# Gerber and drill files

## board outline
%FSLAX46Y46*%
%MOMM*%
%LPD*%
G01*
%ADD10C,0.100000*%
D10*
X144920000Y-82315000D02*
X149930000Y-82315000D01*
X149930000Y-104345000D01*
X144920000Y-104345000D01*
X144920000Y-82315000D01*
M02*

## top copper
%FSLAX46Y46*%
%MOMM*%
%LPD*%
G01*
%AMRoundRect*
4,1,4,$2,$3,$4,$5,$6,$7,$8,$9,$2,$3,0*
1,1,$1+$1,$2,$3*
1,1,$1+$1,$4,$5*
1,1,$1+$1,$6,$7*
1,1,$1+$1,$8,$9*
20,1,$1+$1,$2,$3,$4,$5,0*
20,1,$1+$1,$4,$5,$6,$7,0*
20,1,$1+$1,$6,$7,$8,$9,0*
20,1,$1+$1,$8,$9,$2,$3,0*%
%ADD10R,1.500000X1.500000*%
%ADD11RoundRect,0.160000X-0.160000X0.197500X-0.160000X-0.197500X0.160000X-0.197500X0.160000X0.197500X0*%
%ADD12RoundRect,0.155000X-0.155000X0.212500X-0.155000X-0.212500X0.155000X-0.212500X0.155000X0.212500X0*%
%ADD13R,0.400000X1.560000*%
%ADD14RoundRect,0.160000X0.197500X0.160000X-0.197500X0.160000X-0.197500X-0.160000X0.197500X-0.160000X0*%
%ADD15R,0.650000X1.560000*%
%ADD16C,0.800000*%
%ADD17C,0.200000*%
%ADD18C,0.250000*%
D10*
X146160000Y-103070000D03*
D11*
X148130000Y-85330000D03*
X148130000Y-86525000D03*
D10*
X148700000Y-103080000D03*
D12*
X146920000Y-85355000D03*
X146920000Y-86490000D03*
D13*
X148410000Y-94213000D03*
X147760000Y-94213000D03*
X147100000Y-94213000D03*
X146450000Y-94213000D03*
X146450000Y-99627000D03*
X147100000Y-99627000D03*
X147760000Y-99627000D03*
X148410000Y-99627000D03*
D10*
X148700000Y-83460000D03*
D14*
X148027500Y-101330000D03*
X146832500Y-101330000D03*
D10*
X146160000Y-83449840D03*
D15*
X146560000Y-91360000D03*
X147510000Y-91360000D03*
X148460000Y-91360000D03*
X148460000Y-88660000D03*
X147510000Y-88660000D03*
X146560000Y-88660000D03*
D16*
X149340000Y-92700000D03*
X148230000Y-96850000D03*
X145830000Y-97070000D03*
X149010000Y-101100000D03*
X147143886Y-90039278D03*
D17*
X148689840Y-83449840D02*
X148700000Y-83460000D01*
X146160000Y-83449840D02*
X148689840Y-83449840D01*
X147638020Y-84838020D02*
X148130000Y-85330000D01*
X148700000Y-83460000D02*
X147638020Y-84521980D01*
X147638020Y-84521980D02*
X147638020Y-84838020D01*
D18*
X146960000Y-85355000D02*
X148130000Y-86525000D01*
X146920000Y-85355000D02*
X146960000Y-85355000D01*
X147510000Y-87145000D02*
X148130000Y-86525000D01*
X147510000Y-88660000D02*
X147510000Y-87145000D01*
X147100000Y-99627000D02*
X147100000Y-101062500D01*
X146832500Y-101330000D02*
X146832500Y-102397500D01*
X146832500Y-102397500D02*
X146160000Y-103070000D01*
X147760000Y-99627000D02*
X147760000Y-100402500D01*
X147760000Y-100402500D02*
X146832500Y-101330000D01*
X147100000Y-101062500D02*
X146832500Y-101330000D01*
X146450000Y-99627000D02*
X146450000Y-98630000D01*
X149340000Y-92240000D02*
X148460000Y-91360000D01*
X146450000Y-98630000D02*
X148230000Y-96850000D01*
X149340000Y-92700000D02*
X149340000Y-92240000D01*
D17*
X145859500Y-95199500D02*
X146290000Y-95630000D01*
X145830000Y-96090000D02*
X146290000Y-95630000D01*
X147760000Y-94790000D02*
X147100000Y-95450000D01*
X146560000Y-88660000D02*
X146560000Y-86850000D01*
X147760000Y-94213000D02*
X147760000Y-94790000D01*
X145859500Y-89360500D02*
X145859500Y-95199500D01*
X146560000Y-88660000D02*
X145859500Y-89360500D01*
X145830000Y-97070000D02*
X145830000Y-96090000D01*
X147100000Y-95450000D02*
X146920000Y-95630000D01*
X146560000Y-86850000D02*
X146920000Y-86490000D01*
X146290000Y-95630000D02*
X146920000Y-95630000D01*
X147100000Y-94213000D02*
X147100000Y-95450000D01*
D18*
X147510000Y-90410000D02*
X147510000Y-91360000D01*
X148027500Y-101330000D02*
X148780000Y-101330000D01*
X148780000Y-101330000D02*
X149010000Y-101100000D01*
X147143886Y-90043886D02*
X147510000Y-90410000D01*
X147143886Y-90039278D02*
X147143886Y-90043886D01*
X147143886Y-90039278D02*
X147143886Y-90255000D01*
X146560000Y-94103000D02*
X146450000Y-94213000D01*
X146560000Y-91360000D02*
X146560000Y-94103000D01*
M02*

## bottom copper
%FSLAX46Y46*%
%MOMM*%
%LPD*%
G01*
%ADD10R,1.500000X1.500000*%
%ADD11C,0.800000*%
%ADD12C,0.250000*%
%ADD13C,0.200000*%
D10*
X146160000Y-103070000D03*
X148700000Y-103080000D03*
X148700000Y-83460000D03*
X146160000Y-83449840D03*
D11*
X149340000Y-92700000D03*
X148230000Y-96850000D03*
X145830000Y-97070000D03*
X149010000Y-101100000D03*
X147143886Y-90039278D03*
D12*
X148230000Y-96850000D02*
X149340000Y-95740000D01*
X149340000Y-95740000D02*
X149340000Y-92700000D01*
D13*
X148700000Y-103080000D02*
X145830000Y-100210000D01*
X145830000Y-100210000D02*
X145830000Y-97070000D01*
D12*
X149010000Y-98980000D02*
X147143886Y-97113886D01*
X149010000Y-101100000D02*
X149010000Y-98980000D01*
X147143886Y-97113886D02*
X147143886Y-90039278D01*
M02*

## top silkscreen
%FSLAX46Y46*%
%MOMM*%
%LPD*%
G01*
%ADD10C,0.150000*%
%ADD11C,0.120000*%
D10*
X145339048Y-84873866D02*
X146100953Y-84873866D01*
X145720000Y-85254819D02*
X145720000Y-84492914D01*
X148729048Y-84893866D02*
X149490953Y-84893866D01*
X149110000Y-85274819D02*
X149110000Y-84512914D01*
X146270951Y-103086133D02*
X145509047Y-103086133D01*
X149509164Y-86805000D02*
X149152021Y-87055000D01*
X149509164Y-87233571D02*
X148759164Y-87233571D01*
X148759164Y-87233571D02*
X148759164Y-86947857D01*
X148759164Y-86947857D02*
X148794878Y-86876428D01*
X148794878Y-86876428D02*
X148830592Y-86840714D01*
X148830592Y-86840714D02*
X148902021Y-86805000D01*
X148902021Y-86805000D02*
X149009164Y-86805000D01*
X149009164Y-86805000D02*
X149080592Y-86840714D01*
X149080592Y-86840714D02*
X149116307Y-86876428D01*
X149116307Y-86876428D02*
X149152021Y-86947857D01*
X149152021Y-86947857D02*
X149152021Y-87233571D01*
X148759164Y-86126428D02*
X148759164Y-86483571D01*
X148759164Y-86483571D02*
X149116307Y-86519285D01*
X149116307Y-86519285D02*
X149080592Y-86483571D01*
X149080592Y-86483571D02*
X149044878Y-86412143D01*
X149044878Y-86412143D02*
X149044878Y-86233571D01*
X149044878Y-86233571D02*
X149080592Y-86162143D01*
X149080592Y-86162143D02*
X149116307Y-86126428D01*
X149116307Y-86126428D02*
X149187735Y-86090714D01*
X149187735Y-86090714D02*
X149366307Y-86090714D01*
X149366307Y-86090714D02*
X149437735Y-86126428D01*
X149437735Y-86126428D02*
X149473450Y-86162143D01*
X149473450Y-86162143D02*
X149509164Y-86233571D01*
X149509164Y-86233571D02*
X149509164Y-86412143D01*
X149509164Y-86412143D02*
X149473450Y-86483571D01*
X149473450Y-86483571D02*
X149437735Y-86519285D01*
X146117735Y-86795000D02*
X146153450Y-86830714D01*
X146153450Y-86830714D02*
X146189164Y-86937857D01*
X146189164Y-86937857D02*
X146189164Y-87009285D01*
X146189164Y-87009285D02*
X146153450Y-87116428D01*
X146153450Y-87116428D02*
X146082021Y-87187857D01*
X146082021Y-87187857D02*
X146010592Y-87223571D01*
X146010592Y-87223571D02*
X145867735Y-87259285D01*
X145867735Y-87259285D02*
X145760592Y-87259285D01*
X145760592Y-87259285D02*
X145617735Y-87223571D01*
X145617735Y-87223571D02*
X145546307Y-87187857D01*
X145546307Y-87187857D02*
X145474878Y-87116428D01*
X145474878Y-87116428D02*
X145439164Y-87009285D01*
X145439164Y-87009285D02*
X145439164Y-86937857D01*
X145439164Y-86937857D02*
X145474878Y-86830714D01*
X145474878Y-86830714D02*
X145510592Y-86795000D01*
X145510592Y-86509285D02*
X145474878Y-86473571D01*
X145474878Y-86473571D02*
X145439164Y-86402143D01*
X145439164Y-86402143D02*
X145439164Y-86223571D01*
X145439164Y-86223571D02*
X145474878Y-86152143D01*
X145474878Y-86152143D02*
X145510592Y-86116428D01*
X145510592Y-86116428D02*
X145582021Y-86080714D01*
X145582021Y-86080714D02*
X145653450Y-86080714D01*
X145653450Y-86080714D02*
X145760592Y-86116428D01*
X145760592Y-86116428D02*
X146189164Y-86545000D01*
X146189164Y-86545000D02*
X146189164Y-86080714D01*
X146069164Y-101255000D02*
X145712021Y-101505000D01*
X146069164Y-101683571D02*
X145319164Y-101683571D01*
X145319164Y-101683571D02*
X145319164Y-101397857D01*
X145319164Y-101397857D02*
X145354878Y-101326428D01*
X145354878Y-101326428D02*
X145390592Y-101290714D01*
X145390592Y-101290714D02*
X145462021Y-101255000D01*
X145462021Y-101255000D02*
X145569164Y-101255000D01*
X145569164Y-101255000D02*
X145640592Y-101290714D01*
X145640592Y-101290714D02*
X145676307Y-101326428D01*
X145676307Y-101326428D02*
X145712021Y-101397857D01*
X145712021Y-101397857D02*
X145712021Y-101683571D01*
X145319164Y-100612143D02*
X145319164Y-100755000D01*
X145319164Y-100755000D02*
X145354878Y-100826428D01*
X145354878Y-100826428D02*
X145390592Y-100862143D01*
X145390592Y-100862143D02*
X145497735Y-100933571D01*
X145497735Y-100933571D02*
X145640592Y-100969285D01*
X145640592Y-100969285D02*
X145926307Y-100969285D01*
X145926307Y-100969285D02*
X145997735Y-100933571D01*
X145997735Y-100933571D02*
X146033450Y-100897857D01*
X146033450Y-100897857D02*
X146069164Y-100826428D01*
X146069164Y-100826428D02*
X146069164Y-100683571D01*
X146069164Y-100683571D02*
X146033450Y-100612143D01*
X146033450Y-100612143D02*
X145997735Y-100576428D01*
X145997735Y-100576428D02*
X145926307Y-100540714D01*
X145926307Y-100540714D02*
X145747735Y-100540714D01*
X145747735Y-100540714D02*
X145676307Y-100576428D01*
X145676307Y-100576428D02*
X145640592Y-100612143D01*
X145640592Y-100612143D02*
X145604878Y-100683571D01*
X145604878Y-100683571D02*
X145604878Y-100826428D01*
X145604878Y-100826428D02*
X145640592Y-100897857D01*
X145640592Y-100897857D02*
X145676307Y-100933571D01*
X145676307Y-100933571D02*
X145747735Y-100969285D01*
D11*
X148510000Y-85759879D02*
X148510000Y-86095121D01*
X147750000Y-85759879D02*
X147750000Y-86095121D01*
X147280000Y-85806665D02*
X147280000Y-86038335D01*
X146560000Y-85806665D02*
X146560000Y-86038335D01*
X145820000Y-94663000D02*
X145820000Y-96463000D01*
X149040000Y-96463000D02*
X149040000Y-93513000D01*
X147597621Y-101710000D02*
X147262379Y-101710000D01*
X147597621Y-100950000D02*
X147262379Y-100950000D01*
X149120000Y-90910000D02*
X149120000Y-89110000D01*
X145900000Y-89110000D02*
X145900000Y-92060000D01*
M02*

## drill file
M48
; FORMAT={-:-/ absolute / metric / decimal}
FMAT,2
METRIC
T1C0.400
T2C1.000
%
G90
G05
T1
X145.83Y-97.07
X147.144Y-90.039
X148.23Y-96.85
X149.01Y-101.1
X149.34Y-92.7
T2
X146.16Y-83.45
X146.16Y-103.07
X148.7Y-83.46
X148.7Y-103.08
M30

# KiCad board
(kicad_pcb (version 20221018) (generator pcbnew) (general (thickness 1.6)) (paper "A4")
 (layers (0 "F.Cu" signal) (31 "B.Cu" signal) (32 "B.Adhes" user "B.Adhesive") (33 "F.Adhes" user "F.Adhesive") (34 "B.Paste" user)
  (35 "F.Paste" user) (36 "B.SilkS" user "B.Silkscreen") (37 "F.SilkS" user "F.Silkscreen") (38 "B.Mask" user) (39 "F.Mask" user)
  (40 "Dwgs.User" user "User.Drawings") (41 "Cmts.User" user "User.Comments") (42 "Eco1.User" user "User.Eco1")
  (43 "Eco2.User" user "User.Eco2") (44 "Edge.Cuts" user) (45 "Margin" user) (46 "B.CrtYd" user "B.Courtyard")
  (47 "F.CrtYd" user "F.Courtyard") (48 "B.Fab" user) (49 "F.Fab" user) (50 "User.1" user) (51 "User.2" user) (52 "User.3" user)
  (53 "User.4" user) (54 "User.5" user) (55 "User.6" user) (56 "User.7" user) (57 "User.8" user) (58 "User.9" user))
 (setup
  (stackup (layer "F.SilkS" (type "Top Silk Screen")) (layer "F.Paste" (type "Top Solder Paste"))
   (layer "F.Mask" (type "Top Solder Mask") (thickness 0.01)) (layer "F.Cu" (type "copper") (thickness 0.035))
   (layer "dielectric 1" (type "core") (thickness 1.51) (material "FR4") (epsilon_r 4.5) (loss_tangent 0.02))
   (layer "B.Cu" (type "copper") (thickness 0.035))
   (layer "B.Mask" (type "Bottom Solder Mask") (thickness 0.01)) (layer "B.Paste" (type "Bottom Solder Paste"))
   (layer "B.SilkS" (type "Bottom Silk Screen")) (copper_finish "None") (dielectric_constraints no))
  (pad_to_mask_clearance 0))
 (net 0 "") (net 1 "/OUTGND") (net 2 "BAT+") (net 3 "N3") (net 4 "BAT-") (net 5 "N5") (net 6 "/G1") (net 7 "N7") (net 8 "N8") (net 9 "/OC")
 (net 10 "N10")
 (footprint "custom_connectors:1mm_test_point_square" (layer "F.Cu") (at 146.16 103.08016)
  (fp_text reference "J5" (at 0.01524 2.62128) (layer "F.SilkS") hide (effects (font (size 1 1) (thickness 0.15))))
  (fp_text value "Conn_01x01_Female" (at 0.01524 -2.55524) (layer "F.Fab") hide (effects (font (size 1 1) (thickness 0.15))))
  (pad "1" thru_hole rect (at 0 -0.01016) (size 1.5 1.5) (drill 1) (layers "*.Cu" "*.Mask") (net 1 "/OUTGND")))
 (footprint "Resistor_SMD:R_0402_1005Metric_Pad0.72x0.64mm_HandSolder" (layer "F.Cu") (at 148.13 85.9275 -90)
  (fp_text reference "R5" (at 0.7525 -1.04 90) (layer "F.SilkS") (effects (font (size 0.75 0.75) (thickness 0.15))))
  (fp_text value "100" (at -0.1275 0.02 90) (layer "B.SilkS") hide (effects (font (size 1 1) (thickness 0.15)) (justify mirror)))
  (fp_line (start -0.167621 -0.38) (end 0.167621 -0.38) (stroke (width 0.12) (type solid)) (layer "F.SilkS"))
  (fp_line (start -0.167621 0.38) (end 0.167621 0.38) (stroke (width 0.12) (type solid)) (layer "F.SilkS"))
  (pad "1" smd roundrect (at -0.5975 0 270) (size 0.715 0.64) (layers "F.Cu" "F.Paste" "F.Mask") (roundrect_rratio 0.25) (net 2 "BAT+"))
  (pad "2" smd roundrect (at 0.5975 0 270) (size 0.715 0.64) (layers "F.Cu" "F.Paste" "F.Mask") (roundrect_rratio 0.25) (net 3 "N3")))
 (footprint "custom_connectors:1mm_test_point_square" (layer "F.Cu") (at 148.7 103.09016)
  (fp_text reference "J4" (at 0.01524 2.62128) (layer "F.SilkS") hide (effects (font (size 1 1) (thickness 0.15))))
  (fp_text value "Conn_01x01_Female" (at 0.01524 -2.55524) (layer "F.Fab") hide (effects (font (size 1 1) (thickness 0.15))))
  (pad "1" thru_hole rect (at 0 -0.01016) (size 1.5 1.5) (drill 1) (layers "*.Cu" "*.Mask") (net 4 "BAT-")))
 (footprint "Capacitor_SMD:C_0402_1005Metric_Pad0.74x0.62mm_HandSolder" (layer "F.Cu") (at 146.92 85.9225 -90)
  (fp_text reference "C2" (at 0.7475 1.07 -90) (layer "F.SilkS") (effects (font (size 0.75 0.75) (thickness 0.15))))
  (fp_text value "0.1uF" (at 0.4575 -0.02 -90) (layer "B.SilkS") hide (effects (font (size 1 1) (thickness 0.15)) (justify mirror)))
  (fp_line (start -0.115835 -0.36) (end 0.115835 -0.36) (stroke (width 0.12) (type solid)) (layer "F.SilkS"))
  (fp_line (start -0.115835 0.36) (end 0.115835 0.36) (stroke (width 0.12) (type solid)) (layer "F.SilkS"))
  (pad "1" smd roundrect (at -0.5675 0 270) (size 0.735 0.62) (layers "F.Cu" "F.Paste" "F.Mask") (roundrect_rratio 0.25) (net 3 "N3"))
  (pad "2" smd roundrect (at 0.5675 0 270) (size 0.735 0.62) (layers "F.Cu" "F.Paste" "F.Mask") (roundrect_rratio 0.25) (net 4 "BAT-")))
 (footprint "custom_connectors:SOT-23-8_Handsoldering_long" (layer "F.Cu") (at 147.43 95.563 -90)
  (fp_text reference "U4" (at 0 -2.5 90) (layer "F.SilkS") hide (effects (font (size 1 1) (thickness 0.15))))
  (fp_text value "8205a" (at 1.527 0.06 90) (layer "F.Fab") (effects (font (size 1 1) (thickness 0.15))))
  (fp_line (start -0.9 1.61) (end 0.9 1.61) (stroke (width 0.12) (type solid)) (layer "F.SilkS"))
  (fp_line (start 0.9 -1.61) (end -2.05 -1.61) (stroke (width 0.12) (type solid)) (layer "F.SilkS"))
  (pad "1" smd rect (at -1.35 -0.98 270) (size 1.56 0.4) (layers "F.Cu" "F.Paste" "F.Mask") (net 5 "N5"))
  (pad "2" smd rect (at -1.35 -0.33 270) (size 1.56 0.4) (layers "F.Cu" "F.Paste" "F.Mask") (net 4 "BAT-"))
  (pad "3" smd rect (at -1.35 0.33 270) (size 1.56 0.4) (layers "F.Cu" "F.Paste" "F.Mask") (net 4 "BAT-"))
  (pad "4" smd rect (at -1.35 0.98 270) (size 1.56 0.4) (layers "F.Cu" "F.Paste" "F.Mask") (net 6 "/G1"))
  (pad "5" smd rect (at 4.064 0.98 270) (size 1.56 0.4) (layers "F.Cu" "F.Paste" "F.Mask") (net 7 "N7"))
  (pad "6" smd rect (at 4.064 0.33 270) (size 1.56 0.4) (layers "F.Cu" "F.Paste" "F.Mask") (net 1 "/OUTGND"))
  (pad "7" smd rect (at 4.064 -0.33 270) (size 1.56 0.4) (layers "F.Cu" "F.Paste" "F.Mask") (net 1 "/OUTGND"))
  (pad "8" smd rect (at 4.064 -0.98 270) (size 1.56 0.4) (layers "F.Cu" "F.Paste" "F.Mask") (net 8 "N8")))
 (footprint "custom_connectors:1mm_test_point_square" (layer "F.Cu") (at 148.7 83.47016)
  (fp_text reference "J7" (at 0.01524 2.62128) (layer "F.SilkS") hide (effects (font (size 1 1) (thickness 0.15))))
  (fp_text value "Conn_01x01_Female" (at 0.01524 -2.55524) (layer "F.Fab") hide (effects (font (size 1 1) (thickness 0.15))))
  (pad "1" thru_hole rect (at 0 -0.01016) (size 1.5 1.5) (drill 1) (layers "*.Cu" "*.Mask") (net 2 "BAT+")))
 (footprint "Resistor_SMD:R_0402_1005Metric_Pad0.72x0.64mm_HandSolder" (layer "F.Cu") (at 147.43 101.33 180)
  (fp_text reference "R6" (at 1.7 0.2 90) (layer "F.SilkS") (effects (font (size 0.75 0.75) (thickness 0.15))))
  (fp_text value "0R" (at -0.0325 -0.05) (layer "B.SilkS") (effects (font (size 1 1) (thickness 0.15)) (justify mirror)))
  (fp_line (start -0.167621 -0.38) (end 0.167621 -0.38) (stroke (width 0.12) (type solid)) (layer "F.SilkS"))
  (fp_line (start -0.167621 0.38) (end 0.167621 0.38) (stroke (width 0.12) (type solid)) (layer "F.SilkS"))
  (pad "1" smd roundrect (at -0.5975 0 180) (size 0.715 0.64) (layers "F.Cu" "F.Paste" "F.Mask") (roundrect_rratio 0.25) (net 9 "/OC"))
  (pad "2" smd roundrect (at 0.5975 0 180) (size 0.715 0.64) (layers "F.Cu" "F.Paste" "F.Mask") (roundrect_rratio 0.25) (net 1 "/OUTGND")))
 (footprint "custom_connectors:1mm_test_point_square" (layer "F.Cu") (at 146.16 83.46)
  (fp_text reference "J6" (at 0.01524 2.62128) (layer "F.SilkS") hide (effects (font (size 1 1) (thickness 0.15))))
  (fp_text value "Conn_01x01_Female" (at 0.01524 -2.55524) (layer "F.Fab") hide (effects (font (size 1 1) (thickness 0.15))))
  (pad "1" thru_hole rect (at 0 -0.01016) (size 1.5 1.5) (drill 1) (layers "*.Cu" "*.Mask") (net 2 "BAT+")))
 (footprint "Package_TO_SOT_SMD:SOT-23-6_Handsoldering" (layer "F.Cu") (at 147.51 90.01 90)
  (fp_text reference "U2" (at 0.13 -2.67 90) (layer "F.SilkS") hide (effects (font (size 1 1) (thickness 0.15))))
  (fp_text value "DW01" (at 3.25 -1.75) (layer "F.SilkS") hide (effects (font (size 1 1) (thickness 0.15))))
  (fp_line (start -0.9 1.61) (end 0.9 1.61) (stroke (width 0.12) (type solid)) (layer "F.SilkS"))
  (fp_line (start 0.9 -1.61) (end -2.05 -1.61) (stroke (width 0.12) (type solid)) (layer "F.SilkS"))
  (pad "1" smd rect (at -1.35 -0.95 90) (size 1.56 0.65) (layers "F.Cu" "F.Paste" "F.Mask") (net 6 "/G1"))
  (pad "2" smd rect (at -1.35 0 90) (size 1.56 0.65) (layers "F.Cu" "F.Paste" "F.Mask") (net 9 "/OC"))
  (pad "3" smd rect (at -1.35 0.95 90) (size 1.56 0.65) (layers "F.Cu" "F.Paste" "F.Mask") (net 7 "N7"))
  (pad "4" smd rect (at 1.35 0.95 90) (size 1.56 0.65) (layers "F.Cu" "F.Paste" "F.Mask") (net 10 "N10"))
  (pad "5" smd rect (at 1.35 0 90) (size 1.56 0.65) (layers "F.Cu" "F.Paste" "F.Mask") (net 3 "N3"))
  (pad "6" smd rect (at 1.35 -0.95 90) (size 1.56 0.65) (layers "F.Cu" "F.Paste" "F.Mask") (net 4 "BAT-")))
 (gr_rect (start 144.92 82.315) (end 149.93 104.345) (stroke (width 0.1) (type default)) (fill none) (layer "Edge.Cuts"))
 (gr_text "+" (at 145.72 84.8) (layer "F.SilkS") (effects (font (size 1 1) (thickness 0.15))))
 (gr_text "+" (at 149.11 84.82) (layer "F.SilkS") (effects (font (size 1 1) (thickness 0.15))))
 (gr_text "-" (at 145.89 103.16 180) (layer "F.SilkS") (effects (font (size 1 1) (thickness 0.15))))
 (segment (start 148.68984 83.44984) (end 148.7 83.46) (width 0.2) (layer "F.Cu") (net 2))
 (segment (start 146.16 83.44984) (end 148.68984 83.44984) (width 0.2) (layer "F.Cu") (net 2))
 (segment (start 147.63802 84.83802) (end 148.13 85.33) (width 0.2) (layer "F.Cu") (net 2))
 (segment (start 148.7 83.46) (end 147.63802 84.52198) (width 0.2) (layer "F.Cu") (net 2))
 (segment (start 147.63802 84.52198) (end 147.63802 84.83802) (width 0.2) (layer "F.Cu") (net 2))
 (segment (start 146.96 85.355) (end 148.13 86.525) (width 0.25) (layer "F.Cu") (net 3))
 (segment (start 146.92 85.355) (end 146.96 85.355) (width 0.25) (layer "F.Cu") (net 3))
 (segment (start 147.51 87.145) (end 148.13 86.525) (width 0.25) (layer "F.Cu") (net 3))
 (segment (start 147.51 88.66) (end 147.51 87.145) (width 0.25) (layer "F.Cu") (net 3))
 (segment (start 147.1 99.627) (end 147.1 101.0625) (width 0.25) (layer "F.Cu") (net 1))
 (segment (start 146.8325 101.33) (end 146.8325 102.3975) (width 0.25) (layer "F.Cu") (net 1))
 (segment (start 146.8325 102.3975) (end 146.16 103.07) (width 0.25) (layer "F.Cu") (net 1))
 (segment (start 147.76 99.627) (end 147.76 100.4025) (width 0.25) (layer "F.Cu") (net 1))
 (segment (start 147.76 100.4025) (end 146.8325 101.33) (width 0.25) (layer "F.Cu") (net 1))
 (segment (start 147.1 101.0625) (end 146.8325 101.33) (width 0.25) (layer "F.Cu") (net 1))
 (segment (start 146.45 99.627) (end 146.45 98.63) (width 0.25) (layer "F.Cu") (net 7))
 (segment (start 149.34 92.24) (end 148.46 91.36) (width 0.25) (layer "F.Cu") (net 7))
 (segment (start 146.45 98.63) (end 148.23 96.85) (width 0.25) (layer "F.Cu") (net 7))
 (segment (start 149.34 92.7) (end 149.34 92.24) (width 0.25) (layer "F.Cu") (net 7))
 (via (at 149.34 92.7) (size 0.8) (drill 0.4) (layers "F.Cu" "B.Cu") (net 7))
 (via (at 148.23 96.85) (size 0.8) (drill 0.4) (layers "F.Cu" "B.Cu") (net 7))
 (segment (start 148.23 96.85) (end 149.34 95.74) (width 0.25) (layer "B.Cu") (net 7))
 (segment (start 149.34 95.74) (end 149.34 92.7) (width 0.25) (layer "B.Cu") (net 7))
 (segment (start 145.8595 95.1995) (end 146.29 95.63) (width 0.2) (layer "F.Cu") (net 4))
 (segment (start 145.83 96.09) (end 146.29 95.63) (width 0.2) (layer "F.Cu") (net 4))
 (segment (start 147.76 94.79) (end 147.1 95.45) (width 0.2) (layer "F.Cu") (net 4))
 (segment (start 146.56 88.66) (end 146.56 86.85) (width 0.2) (layer "F.Cu") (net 4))
 (segment (start 147.76 94.213) (end 147.76 94.79) (width 0.2) (layer "F.Cu") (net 4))
 (segment (start 145.8595 89.3605) (end 145.8595 95.1995) (width 0.2) (layer "F.Cu") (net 4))
 (segment (start 146.56 88.66) (end 145.8595 89.3605) (width 0.2) (layer "F.Cu") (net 4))
 (segment (start 145.83 97.07) (end 145.83 96.09) (width 0.2) (layer "F.Cu") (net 4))
 (segment (start 147.1 95.45) (end 146.92 95.63) (width 0.2) (layer "F.Cu") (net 4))
 (segment (start 146.56 86.85) (end 146.92 86.49) (width 0.2) (layer "F.Cu") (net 4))
 (segment (start 146.29 95.63) (end 146.92 95.63) (width 0.2) (layer "F.Cu") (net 4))
 (segment (start 147.1 94.213) (end 147.1 95.45) (width 0.2) (layer "F.Cu") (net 4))
 (via (at 145.83 97.07) (size 0.8) (drill 0.4) (layers "F.Cu" "B.Cu") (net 4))
 (segment (start 148.7 103.08) (end 145.83 100.21) (width 0.2) (layer "B.Cu") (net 4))
 (segment (start 145.83 100.21) (end 145.83 97.07) (width 0.2) (layer "B.Cu") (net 4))
 (segment (start 147.51 90.41) (end 147.51 91.36) (width 0.25) (layer "F.Cu") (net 9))
 (segment (start 148.0275 101.33) (end 148.78 101.33) (width 0.25) (layer "F.Cu") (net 9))
 (segment (start 148.78 101.33) (end 149.01 101.1) (width 0.25) (layer "F.Cu") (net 9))
 (segment (start 147.143886 90.043886) (end 147.51 90.41) (width 0.25) (layer "F.Cu") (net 9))
 (segment (start 147.143886 90.039278) (end 147.143886 90.043886) (width 0.25) (layer "F.Cu") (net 9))
 (segment (start 147.143886 90.039278) (end 147.143886 90.255) (width 0.25) (layer "F.Cu") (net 9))
 (via (at 149.01 101.1) (size 0.8) (drill 0.4) (layers "F.Cu" "B.Cu") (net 9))
 (via (at 147.143886 90.039278) (size 0.8) (drill 0.4) (layers "F.Cu" "B.Cu") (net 9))
 (segment (start 149.01 98.98) (end 147.143886 97.113886) (width 0.25) (layer "B.Cu") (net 9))
 (segment (start 149.01 101.1) (end 149.01 98.98) (width 0.25) (layer "B.Cu") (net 9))
 (segment (start 147.143886 97.113886) (end 147.143886 90.039278) (width 0.25) (layer "B.Cu") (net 9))
 (segment (start 146.56 94.103) (end 146.45 94.213) (width 0.25) (layer "F.Cu") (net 6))
 (segment (start 146.56 91.36) (end 146.56 94.103) (width 0.25) (layer "F.Cu") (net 6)))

